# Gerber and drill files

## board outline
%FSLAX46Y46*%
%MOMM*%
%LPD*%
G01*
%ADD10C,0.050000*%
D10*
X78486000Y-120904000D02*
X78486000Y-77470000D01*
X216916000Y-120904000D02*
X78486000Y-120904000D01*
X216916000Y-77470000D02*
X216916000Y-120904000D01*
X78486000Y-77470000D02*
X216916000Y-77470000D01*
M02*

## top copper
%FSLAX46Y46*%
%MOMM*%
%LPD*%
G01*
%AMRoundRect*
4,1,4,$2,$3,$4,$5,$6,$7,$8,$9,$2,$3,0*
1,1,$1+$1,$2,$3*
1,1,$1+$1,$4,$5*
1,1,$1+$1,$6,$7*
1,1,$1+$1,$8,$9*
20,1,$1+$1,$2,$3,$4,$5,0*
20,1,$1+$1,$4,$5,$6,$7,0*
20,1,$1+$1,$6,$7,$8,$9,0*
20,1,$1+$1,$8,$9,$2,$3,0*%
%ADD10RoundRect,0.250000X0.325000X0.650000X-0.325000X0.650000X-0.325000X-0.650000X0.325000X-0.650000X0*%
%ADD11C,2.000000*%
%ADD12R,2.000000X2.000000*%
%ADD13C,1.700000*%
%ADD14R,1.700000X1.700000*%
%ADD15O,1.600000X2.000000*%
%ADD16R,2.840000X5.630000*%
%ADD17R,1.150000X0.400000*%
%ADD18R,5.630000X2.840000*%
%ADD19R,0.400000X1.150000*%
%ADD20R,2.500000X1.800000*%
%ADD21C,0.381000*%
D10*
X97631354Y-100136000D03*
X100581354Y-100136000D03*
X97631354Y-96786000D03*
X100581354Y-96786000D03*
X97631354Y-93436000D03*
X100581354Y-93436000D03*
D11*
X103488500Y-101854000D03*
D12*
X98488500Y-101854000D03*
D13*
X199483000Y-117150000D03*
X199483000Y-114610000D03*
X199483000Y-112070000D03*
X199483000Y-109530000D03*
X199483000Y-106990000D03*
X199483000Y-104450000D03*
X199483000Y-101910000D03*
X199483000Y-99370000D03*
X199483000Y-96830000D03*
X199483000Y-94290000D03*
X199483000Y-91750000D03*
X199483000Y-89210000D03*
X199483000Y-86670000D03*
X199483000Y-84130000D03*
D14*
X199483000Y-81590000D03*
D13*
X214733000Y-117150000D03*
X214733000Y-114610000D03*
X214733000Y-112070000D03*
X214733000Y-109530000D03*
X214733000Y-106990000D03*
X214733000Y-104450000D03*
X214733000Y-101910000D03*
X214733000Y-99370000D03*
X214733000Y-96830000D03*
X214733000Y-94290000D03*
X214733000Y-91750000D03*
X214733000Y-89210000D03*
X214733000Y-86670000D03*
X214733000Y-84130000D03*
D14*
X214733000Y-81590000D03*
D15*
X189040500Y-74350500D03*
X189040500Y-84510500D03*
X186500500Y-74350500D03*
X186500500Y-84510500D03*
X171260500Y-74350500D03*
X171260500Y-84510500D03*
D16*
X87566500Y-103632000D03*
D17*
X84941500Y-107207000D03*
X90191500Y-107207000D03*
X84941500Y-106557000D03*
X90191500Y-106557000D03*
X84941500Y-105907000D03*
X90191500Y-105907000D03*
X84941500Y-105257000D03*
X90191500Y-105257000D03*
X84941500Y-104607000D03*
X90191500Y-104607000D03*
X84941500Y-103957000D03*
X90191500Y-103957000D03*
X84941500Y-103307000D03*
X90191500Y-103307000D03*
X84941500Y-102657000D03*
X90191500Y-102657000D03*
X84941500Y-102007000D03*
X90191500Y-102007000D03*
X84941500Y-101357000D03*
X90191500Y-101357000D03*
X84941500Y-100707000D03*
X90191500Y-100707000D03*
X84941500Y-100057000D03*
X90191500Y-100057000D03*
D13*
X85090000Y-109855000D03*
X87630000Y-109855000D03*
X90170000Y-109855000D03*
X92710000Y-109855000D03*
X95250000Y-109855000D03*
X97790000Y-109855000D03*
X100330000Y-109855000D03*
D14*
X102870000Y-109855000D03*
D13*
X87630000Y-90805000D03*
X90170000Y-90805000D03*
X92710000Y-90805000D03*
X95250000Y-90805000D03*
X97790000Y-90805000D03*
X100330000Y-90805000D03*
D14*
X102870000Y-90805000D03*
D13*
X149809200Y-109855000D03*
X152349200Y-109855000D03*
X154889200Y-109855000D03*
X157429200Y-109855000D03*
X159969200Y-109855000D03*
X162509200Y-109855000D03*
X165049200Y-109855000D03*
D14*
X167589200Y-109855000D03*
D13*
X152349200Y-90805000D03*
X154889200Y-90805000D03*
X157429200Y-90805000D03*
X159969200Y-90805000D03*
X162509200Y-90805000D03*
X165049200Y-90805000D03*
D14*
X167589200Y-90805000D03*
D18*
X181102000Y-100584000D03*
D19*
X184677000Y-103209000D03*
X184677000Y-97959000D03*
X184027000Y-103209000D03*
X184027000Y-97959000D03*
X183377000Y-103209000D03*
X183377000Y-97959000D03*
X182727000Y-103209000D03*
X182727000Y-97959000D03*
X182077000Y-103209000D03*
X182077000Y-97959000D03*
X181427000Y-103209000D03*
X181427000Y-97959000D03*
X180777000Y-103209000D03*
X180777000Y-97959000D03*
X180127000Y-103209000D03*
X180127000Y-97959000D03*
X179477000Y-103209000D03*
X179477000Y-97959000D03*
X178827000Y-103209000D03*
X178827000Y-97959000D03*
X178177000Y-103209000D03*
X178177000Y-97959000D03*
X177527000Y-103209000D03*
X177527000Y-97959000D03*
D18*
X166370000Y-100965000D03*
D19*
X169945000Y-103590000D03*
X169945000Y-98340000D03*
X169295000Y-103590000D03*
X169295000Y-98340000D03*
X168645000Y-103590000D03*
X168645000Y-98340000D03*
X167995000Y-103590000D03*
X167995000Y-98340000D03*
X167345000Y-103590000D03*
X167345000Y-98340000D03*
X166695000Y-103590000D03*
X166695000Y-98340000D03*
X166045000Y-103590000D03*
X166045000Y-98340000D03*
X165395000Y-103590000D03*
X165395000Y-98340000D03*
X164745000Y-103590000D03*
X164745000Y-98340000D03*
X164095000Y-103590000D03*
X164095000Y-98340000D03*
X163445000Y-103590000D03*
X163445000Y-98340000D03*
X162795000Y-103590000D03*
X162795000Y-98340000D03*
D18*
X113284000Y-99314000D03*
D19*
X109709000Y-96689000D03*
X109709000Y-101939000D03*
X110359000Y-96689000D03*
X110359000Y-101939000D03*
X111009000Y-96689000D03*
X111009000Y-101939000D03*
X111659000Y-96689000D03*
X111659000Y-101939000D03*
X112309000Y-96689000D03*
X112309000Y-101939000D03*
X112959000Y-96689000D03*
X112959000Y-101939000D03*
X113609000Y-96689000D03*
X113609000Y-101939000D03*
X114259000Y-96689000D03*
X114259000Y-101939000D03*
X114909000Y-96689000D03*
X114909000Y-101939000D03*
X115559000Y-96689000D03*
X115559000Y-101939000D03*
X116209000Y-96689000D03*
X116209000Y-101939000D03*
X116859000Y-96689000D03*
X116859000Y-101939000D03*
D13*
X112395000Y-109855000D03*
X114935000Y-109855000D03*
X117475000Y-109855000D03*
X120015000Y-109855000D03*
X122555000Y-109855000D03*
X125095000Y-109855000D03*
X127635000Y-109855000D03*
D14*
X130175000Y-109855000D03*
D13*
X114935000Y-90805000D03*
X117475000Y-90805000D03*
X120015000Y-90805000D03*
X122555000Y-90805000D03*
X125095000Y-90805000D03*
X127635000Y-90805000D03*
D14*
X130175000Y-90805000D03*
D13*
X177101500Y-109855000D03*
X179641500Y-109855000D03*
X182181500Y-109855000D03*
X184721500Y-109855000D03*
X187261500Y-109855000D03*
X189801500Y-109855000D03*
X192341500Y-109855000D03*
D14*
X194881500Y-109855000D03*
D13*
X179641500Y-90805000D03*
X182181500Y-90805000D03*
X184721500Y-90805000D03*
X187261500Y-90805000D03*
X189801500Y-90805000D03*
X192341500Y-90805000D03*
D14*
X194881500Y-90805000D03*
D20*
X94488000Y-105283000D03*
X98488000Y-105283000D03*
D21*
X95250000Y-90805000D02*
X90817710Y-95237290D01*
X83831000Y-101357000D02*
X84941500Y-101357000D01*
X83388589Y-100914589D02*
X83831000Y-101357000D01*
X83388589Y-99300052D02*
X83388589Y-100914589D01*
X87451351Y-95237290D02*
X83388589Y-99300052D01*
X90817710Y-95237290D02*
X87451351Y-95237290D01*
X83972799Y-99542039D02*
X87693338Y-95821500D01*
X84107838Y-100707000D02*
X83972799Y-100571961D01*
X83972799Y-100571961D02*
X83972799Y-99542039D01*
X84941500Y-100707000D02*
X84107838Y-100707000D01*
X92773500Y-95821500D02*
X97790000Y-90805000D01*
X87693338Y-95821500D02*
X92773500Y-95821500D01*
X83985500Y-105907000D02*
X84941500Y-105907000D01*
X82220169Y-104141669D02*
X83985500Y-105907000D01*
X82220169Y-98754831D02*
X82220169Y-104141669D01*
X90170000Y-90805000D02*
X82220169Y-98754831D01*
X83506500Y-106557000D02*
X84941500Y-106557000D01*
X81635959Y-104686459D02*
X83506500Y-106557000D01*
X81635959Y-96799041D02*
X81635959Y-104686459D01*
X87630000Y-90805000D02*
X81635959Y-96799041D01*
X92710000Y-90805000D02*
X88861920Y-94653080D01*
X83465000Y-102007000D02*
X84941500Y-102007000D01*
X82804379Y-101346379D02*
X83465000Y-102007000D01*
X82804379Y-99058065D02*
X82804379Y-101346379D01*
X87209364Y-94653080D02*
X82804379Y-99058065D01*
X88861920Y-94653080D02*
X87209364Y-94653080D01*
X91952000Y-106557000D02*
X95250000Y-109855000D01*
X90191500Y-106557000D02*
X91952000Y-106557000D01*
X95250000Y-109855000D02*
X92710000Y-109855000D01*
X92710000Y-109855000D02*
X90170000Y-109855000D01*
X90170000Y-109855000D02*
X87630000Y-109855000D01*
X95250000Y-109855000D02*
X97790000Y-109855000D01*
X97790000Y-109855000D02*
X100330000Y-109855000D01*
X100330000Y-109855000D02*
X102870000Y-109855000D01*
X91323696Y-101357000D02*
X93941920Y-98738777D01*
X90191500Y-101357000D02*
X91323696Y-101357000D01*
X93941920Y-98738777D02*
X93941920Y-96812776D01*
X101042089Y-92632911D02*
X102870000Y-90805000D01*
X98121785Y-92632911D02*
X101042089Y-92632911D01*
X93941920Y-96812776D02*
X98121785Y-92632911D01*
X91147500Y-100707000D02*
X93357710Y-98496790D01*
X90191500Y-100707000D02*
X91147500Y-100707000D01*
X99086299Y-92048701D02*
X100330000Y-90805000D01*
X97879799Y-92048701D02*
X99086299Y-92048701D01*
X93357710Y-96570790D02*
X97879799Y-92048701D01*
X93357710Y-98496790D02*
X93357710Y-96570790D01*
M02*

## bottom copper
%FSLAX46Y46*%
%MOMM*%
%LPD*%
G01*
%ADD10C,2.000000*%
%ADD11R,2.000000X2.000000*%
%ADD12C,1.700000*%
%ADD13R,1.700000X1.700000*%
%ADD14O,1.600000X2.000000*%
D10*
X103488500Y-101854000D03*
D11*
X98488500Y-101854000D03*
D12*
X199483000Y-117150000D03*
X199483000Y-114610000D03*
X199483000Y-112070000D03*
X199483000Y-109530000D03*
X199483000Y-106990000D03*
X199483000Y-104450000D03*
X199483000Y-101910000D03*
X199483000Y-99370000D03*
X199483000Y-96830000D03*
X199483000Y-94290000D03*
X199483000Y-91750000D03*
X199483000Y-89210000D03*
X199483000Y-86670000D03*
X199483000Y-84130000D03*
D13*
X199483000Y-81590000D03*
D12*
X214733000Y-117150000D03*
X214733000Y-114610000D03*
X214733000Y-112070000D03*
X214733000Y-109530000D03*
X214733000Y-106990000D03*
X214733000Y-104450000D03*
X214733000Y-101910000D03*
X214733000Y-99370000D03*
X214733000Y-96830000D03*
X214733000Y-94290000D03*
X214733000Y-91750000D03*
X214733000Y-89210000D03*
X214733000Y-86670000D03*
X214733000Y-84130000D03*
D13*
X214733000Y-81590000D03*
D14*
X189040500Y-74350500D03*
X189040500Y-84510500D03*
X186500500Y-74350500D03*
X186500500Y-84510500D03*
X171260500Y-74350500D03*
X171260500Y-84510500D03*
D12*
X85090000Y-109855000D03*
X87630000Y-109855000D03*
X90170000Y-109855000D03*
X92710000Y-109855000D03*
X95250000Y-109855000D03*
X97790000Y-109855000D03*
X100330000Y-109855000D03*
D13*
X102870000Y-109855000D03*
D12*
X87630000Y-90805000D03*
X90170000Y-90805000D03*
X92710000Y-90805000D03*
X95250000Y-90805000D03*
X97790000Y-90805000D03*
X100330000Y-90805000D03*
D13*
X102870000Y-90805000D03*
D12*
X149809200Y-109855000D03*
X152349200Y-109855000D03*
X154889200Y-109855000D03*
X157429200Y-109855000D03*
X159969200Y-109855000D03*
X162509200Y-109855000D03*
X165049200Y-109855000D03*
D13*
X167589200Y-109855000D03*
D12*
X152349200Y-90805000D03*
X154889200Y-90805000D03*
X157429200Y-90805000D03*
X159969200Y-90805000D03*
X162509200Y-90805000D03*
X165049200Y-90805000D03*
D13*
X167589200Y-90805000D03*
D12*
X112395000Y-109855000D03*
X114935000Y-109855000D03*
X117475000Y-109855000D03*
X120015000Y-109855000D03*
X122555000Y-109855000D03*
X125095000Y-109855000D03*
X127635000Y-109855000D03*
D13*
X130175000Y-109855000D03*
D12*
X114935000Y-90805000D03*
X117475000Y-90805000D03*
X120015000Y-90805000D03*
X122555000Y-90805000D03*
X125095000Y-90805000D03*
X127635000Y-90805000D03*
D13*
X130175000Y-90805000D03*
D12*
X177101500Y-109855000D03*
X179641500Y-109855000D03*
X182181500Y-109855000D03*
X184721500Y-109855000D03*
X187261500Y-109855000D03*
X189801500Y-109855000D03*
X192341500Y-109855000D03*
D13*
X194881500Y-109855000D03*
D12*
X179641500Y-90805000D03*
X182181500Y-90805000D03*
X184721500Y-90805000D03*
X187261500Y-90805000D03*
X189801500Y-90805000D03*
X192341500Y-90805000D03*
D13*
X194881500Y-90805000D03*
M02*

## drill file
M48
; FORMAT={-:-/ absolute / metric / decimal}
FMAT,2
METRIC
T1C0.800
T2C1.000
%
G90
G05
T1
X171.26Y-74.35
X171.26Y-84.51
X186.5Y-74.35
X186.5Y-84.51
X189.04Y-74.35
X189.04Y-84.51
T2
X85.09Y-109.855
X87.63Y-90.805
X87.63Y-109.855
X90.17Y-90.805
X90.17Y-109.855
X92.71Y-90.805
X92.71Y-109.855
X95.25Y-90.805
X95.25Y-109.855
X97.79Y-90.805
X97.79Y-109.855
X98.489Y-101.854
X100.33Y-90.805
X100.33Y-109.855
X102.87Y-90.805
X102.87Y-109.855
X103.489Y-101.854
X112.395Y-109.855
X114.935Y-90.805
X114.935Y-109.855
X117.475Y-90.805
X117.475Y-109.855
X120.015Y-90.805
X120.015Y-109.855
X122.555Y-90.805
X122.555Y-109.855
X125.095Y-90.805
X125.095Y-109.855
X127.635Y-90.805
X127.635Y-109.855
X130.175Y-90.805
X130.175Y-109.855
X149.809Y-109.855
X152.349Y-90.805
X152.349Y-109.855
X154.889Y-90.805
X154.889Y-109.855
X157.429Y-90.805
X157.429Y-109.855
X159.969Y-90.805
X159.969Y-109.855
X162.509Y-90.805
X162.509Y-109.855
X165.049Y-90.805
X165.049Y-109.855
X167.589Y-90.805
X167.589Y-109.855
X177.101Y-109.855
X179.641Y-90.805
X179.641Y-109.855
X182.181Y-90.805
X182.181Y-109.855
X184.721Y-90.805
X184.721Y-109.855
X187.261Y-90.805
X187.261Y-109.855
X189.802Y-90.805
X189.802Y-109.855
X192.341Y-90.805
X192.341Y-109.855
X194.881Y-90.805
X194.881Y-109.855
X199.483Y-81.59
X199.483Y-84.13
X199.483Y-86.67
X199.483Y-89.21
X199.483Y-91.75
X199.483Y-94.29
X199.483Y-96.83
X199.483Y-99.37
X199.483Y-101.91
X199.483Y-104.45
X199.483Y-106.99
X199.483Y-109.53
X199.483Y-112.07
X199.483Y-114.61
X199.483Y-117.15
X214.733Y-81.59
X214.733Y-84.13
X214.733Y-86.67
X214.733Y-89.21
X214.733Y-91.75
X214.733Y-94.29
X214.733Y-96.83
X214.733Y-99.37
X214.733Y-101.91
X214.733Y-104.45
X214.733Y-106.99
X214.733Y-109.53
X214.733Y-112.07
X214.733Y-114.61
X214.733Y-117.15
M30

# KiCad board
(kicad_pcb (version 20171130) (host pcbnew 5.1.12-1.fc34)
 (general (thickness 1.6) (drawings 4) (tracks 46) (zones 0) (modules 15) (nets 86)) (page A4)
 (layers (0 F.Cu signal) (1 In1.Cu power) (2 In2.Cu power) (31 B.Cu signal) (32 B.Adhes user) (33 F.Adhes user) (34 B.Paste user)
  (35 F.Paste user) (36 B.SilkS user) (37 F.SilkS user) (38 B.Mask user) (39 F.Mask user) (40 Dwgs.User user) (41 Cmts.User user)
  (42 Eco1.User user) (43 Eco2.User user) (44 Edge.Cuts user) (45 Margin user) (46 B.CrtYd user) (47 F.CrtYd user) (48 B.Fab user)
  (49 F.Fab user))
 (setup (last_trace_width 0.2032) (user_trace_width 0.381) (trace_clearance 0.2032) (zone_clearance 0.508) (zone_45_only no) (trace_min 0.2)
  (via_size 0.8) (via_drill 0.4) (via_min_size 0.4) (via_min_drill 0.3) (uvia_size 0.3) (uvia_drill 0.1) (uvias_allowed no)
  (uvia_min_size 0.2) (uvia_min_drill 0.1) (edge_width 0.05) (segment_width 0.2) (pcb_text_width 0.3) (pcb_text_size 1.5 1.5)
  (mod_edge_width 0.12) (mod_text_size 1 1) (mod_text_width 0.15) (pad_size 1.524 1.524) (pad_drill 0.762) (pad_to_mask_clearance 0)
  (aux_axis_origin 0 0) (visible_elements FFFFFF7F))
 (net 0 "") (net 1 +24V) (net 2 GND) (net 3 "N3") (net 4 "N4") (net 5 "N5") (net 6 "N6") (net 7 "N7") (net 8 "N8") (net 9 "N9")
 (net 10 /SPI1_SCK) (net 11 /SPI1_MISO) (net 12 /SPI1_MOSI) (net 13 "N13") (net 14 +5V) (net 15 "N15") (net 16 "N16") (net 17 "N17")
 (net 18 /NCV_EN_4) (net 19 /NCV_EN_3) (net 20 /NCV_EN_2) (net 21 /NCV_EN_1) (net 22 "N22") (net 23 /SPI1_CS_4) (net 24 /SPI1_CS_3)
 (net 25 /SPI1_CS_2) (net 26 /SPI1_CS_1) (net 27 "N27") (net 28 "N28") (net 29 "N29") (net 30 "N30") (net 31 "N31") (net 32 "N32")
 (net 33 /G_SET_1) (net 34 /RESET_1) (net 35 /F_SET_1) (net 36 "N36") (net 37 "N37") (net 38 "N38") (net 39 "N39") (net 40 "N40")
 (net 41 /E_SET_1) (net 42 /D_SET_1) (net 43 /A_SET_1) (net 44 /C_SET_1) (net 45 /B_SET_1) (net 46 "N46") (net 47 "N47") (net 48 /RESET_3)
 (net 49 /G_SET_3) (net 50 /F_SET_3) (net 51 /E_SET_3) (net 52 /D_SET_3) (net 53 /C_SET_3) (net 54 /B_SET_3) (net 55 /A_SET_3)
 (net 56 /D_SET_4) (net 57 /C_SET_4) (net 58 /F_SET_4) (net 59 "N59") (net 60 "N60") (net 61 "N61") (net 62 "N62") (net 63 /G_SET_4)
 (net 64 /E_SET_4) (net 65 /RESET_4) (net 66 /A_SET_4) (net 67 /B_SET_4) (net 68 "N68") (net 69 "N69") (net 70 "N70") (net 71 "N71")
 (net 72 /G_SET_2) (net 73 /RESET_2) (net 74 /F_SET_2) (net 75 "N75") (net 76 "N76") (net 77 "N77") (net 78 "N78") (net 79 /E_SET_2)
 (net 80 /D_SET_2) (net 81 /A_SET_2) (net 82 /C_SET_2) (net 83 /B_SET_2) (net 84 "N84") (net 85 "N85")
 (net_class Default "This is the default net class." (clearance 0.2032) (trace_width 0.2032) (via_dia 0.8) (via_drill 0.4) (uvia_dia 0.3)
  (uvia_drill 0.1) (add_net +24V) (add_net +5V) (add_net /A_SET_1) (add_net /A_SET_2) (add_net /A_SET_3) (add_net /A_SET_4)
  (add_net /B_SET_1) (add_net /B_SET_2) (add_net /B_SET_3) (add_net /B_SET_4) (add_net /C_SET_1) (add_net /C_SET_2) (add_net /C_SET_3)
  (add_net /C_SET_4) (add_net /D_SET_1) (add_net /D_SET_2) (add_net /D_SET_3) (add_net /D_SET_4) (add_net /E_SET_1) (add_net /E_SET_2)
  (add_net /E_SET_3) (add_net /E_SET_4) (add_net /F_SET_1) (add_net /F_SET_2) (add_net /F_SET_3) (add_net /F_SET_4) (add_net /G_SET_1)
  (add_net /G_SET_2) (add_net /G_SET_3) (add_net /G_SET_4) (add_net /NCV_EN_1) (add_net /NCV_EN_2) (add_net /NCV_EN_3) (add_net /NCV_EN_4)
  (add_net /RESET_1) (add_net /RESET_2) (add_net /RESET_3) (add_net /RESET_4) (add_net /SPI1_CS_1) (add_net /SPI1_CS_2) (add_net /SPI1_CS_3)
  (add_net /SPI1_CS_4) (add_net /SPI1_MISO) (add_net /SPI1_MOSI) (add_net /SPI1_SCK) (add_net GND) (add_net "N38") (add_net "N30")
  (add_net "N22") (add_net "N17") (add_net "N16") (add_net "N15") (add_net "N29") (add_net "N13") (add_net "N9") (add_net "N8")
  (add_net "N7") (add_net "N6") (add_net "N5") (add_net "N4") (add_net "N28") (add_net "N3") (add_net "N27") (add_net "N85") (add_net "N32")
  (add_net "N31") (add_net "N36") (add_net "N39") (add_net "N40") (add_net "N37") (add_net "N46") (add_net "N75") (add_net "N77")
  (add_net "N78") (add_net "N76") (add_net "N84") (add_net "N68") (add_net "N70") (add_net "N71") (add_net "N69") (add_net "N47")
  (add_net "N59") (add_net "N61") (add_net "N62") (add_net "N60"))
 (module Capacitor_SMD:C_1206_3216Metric (layer F.Cu) (at 99.106354 100.136 180)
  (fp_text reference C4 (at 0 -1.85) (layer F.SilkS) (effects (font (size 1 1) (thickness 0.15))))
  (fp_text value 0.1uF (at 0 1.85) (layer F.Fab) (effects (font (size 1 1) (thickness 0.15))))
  (pad 2 smd roundrect (at 1.475 0 180) (size 1.15 1.8) (layers F.Cu F.Paste F.Mask) (roundrect_rratio 0.217391) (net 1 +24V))
  (pad 1 smd roundrect (at -1.475 0 180) (size 1.15 1.8) (layers F.Cu F.Paste F.Mask) (roundrect_rratio 0.217391) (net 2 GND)))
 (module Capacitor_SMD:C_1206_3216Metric (layer F.Cu) (at 99.106354 96.786 180)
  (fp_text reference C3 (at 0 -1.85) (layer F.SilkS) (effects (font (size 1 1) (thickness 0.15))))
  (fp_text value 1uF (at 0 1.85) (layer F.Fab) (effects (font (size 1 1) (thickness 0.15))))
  (pad 2 smd roundrect (at 1.475 0 180) (size 1.15 1.8) (layers F.Cu F.Paste F.Mask) (roundrect_rratio 0.217391) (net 1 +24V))
  (pad 1 smd roundrect (at -1.475 0 180) (size 1.15 1.8) (layers F.Cu F.Paste F.Mask) (roundrect_rratio 0.217391) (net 2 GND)))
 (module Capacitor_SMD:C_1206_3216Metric (layer F.Cu) (at 99.106354 93.436 180)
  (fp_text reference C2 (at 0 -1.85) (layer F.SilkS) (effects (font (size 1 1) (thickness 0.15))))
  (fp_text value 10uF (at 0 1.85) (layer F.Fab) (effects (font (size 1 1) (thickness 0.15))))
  (pad 2 smd roundrect (at 1.475 0 180) (size 1.15 1.8) (layers F.Cu F.Paste F.Mask) (roundrect_rratio 0.217391) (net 1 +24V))
  (pad 1 smd roundrect (at -1.475 0 180) (size 1.15 1.8) (layers F.Cu F.Paste F.Mask) (roundrect_rratio 0.217391) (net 2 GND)))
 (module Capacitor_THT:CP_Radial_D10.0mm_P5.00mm (layer B.Cu) (at 98.4885 101.854)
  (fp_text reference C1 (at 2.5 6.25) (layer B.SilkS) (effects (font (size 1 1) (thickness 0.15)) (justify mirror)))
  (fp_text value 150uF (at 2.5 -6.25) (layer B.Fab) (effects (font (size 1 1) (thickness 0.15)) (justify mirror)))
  (pad 2 thru_hole circle (at 5 0) (size 2 2) (drill 1) (layers *.Cu *.Mask) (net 2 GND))
  (pad 1 thru_hole rect (at 0 0) (size 2 2) (drill 1) (layers *.Cu *.Mask) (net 1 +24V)))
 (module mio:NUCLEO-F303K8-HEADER (layer B.Cu) (at 216.408 123.19 180)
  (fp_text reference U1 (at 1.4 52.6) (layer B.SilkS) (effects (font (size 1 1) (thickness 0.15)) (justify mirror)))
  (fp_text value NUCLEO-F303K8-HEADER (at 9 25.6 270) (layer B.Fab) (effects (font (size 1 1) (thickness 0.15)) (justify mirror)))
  (pad 30 thru_hole circle (at 16.925 6.04 180) (size 1.7 1.7) (drill 1) (layers *.Cu *.Mask) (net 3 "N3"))
  (pad 29 thru_hole circle (at 16.925 8.58 180) (size 1.7 1.7) (drill 1) (layers *.Cu *.Mask) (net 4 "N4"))
  (pad 28 thru_hole circle (at 16.925 11.12 180) (size 1.7 1.7) (drill 1) (layers *.Cu *.Mask) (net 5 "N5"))
  (pad 27 thru_hole circle (at 16.925 13.66 180) (size 1.7 1.7) (drill 1) (layers *.Cu *.Mask) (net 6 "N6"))
  (pad 26 thru_hole circle (at 16.925 16.2 180) (size 1.7 1.7) (drill 1) (layers *.Cu *.Mask) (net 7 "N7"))
  (pad 25 thru_hole circle (at 16.925 18.74 180) (size 1.7 1.7) (drill 1) (layers *.Cu *.Mask) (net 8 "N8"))
  (pad 24 thru_hole circle (at 16.925 21.28 180) (size 1.7 1.7) (drill 1) (layers *.Cu *.Mask) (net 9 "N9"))
  (pad 23 thru_hole circle (at 16.925 23.82 180) (size 1.7 1.7) (drill 1) (layers *.Cu *.Mask) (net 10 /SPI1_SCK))
  (pad 22 thru_hole circle (at 16.925 26.36 180) (size 1.7 1.7) (drill 1) (layers *.Cu *.Mask) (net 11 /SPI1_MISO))
  (pad 21 thru_hole circle (at 16.925 28.9 180) (size 1.7 1.7) (drill 1) (layers *.Cu *.Mask) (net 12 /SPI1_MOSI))
  (pad 20 thru_hole circle (at 16.925 31.44 180) (size 1.7 1.7) (drill 1) (layers *.Cu *.Mask) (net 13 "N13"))
  (pad 19 thru_hole circle (at 16.925 33.98 180) (size 1.7 1.7) (drill 1) (layers *.Cu *.Mask) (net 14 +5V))
  (pad 18 thru_hole circle (at 16.925 36.52 180) (size 1.7 1.7) (drill 1) (layers *.Cu *.Mask) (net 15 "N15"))
  (pad 17 thru_hole circle (at 16.925 39.06 180) (size 1.7 1.7) (drill 1) (layers *.Cu *.Mask) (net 2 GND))
  (pad 16 thru_hole rect (at 16.925 41.6 180) (size 1.7 1.7) (drill 1) (layers *.Cu *.Mask) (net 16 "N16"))
  (pad 15 thru_hole circle (at 1.675 6.04 180) (size 1.7 1.7) (drill 1) (layers *.Cu *.Mask) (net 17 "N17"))
  (pad 14 thru_hole circle (at 1.675 8.58 180) (size 1.7 1.7) (drill 1) (layers *.Cu *.Mask) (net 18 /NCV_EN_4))
  (pad 13 thru_hole circle (at 1.675 11.12 180) (size 1.7 1.7) (drill 1) (layers *.Cu *.Mask) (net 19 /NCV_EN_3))
  (pad 12 thru_hole circle (at 1.675 13.66 180) (size 1.7 1.7) (drill 1) (layers *.Cu *.Mask) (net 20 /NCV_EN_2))
  (pad 11 thru_hole circle (at 1.675 16.2 180) (size 1.7 1.7) (drill 1) (layers *.Cu *.Mask) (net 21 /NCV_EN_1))
  (pad 10 thru_hole circle (at 1.675 18.74 180) (size 1.7 1.7) (drill 1) (layers *.Cu *.Mask) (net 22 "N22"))
  (pad 9 thru_hole circle (at 1.675 21.28 180) (size 1.7 1.7) (drill 1) (layers *.Cu *.Mask) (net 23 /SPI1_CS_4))
  (pad 8 thru_hole circle (at 1.675 23.82 180) (size 1.7 1.7) (drill 1) (layers *.Cu *.Mask) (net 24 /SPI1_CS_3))
  (pad 7 thru_hole circle (at 1.675 26.36 180) (size 1.7 1.7) (drill 1) (layers *.Cu *.Mask) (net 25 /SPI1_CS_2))
  (pad 6 thru_hole circle (at 1.675 28.9 180) (size 1.7 1.7) (drill 1) (layers *.Cu *.Mask) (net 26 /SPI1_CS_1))
  (pad 5 thru_hole circle (at 1.675 31.44 180) (size 1.7 1.7) (drill 1) (layers *.Cu *.Mask) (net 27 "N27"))
  (pad 4 thru_hole circle (at 1.675 33.98 180) (size 1.7 1.7) (drill 1) (layers *.Cu *.Mask) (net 2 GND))
  (pad 3 thru_hole circle (at 1.675 36.52 180) (size 1.7 1.7) (drill 1) (layers *.Cu *.Mask) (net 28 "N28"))
  (pad 2 thru_hole circle (at 1.675 39.06 180) (size 1.7 1.7) (drill 1) (layers *.Cu *.Mask) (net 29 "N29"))
  (pad 1 thru_hole rect (at 1.675 41.6 180) (size 1.7 1.7) (drill 1) (layers *.Cu *.Mask) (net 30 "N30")))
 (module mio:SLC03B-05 (layer B.Cu) (at 169.1005 72.5805)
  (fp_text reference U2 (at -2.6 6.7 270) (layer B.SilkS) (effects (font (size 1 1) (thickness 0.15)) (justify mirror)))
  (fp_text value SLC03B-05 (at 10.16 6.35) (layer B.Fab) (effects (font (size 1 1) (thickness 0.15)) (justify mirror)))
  (pad 8 thru_hole oval (at 19.94 1.77) (size 1.6 2) (drill 0.8) (layers *.Cu *.Mask) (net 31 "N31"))
  (pad 9 thru_hole oval (at 19.94 11.93) (size 1.6 2) (drill 0.8) (layers *.Cu *.Mask) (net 14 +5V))
  (pad 7 thru_hole oval (at 17.4 1.77) (size 1.6 2) (drill 0.8) (layers *.Cu *.Mask) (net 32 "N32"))
  (pad 10 thru_hole oval (at 17.4 11.93) (size 1.6 2) (drill 0.8) (layers *.Cu *.Mask) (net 2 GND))
  (pad 1 thru_hole oval (at 2.16 1.77) (size 1.6 2) (drill 0.8) (layers *.Cu *.Mask) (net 2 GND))
  (pad 16 thru_hole oval (at 2.16 11.93) (size 1.6 2) (drill 0.8) (layers *.Cu *.Mask) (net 1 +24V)))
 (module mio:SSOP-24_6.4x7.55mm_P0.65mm (layer F.Cu) (at 87.5665 103.632 270)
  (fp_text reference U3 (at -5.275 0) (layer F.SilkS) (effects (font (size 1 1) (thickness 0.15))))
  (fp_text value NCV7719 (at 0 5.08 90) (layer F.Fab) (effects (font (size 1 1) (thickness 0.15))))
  (pad 25 smd rect (at 0 0 270) (size 5.63 2.84) (layers F.Cu F.Paste F.Mask) (zone_connect 1) (thermal_width 0.5) (thermal_gap 0.5))
  (pad 12 smd rect (at 3.575 2.625 270) (size 0.4 1.15) (layers F.Cu F.Paste F.Mask) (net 2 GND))
  (pad 13 smd rect (at 3.575 -2.625 270) (size 0.4 1.15) (layers F.Cu F.Paste F.Mask) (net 2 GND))
  (pad 11 smd rect (at 2.925 2.625 270) (size 0.4 1.15) (layers F.Cu F.Paste F.Mask) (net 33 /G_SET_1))
  (pad 14 smd rect (at 2.925 -2.625 270) (size 0.4 1.15) (layers F.Cu F.Paste F.Mask) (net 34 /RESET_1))
  (pad 10 smd rect (at 2.275 2.625 270) (size 0.4 1.15) (layers F.Cu F.Paste F.Mask) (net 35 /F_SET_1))
  (pad 15 smd rect (at 2.275 -2.625 270) (size 0.4 1.15) (layers F.Cu F.Paste F.Mask) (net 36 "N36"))
  (pad 9 smd rect (at 1.625 2.625 270) (size 0.4 1.15) (layers F.Cu F.Paste F.Mask) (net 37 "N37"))
  (pad 16 smd rect (at 1.625 -2.625 270) (size 0.4 1.15) (layers F.Cu F.Paste F.Mask) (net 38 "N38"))
  (pad 8 smd rect (at 0.975 2.625 270) (size 0.4 1.15) (layers F.Cu F.Paste F.Mask) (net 21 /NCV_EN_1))
  (pad 17 smd rect (at 0.975 -2.625 270) (size 0.4 1.15) (layers F.Cu F.Paste F.Mask) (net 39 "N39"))
  (pad 7 smd rect (at 0.325 2.625 270) (size 0.4 1.15) (layers F.Cu F.Paste F.Mask) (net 11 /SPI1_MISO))
  (pad 18 smd rect (at 0.325 -2.625 270) (size 0.4 1.15) (layers F.Cu F.Paste F.Mask) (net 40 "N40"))
  (pad 6 smd rect (at -0.325 2.625 270) (size 0.4 1.15) (layers F.Cu F.Paste F.Mask) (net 14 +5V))
  (pad 19 smd rect (at -0.325 -2.625 270) (size 0.4 1.15) (layers F.Cu F.Paste F.Mask) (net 26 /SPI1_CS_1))
  (pad 5 smd rect (at -0.975 2.625 270) (size 0.4 1.15) (layers F.Cu F.Paste F.Mask) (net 12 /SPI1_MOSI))
  (pad 20 smd rect (at -0.975 -2.625 270) (size 0.4 1.15) (layers F.Cu F.Paste F.Mask) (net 10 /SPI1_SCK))
  (pad 4 smd rect (at -1.625 2.625 270) (size 0.4 1.15) (layers F.Cu F.Paste F.Mask) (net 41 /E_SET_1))
  (pad 21 smd rect (at -1.625 -2.625 270) (size 0.4 1.15) (layers F.Cu F.Paste F.Mask) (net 38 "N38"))
  (pad 3 smd rect (at -2.275 2.625 270) (size 0.4 1.15) (layers F.Cu F.Paste F.Mask) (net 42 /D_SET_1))
  (pad 22 smd rect (at -2.275 -2.625 270) (size 0.4 1.15) (layers F.Cu F.Paste F.Mask) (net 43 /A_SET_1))
  (pad 2 smd rect (at -2.925 2.625 270) (size 0.4 1.15) (layers F.Cu F.Paste F.Mask) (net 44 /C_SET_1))
  (pad 23 smd rect (at -2.925 -2.625 270) (size 0.4 1.15) (layers F.Cu F.Paste F.Mask) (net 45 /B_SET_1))
  (pad 1 smd rect (at -3.575 2.625 270) (size 0.4 1.15) (layers F.Cu F.Paste F.Mask) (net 2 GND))
  (pad 24 smd rect (at -3.575 -2.625 270) (size 0.4 1.15) (layers F.Cu F.Paste F.Mask) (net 2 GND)))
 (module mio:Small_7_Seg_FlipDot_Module (layer F.Cu) (at 81.28 116.205)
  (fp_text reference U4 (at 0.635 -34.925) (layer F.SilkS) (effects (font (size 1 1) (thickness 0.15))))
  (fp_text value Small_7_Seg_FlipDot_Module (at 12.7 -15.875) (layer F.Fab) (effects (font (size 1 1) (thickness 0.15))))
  (pad 15 thru_hole circle (at 3.81 -6.35) (size 1.7 1.7) (drill 1) (layers *.Cu *.Mask) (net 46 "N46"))
  (pad 14 thru_hole circle (at 6.35 -6.35) (size 1.7 1.7) (drill 1) (layers *.Cu *.Mask) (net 34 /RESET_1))
  (pad 13 thru_hole circle (at 8.89 -6.35) (size 1.7 1.7) (drill 1) (layers *.Cu *.Mask) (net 34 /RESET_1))
  (pad 12 thru_hole circle (at 11.43 -6.35) (size 1.7 1.7) (drill 1) (layers *.Cu *.Mask) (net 34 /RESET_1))
  (pad 11 thru_hole circle (at 13.97 -6.35) (size 1.7 1.7) (drill 1) (layers *.Cu *.Mask) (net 34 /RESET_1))
  (pad 10 thru_hole circle (at 16.51 -6.35) (size 1.7 1.7) (drill 1) (layers *.Cu *.Mask) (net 34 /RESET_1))
  (pad 9 thru_hole circle (at 19.05 -6.35) (size 1.7 1.7) (drill 1) (layers *.Cu *.Mask) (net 34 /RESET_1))
  (pad 8 thru_hole rect (at 21.59 -6.35) (size 1.7 1.7) (drill 1) (layers *.Cu *.Mask) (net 34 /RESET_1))
  (pad 7 thru_hole circle (at 6.35 -25.4) (size 1.7 1.7) (drill 1) (layers *.Cu *.Mask) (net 33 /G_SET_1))
  (pad 6 thru_hole circle (at 8.89 -25.4) (size 1.7 1.7) (drill 1) (layers *.Cu *.Mask) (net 35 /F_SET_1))
  (pad 5 thru_hole circle (at 11.43 -25.4) (size 1.7 1.7) (drill 1) (layers *.Cu *.Mask) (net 41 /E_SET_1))
  (pad 4 thru_hole circle (at 13.97 -25.4) (size 1.7 1.7) (drill 1) (layers *.Cu *.Mask) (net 42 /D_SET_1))
  (pad 3 thru_hole circle (at 16.51 -25.4) (size 1.7 1.7) (drill 1) (layers *.Cu *.Mask) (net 44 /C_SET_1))
  (pad 2 thru_hole circle (at 19.05 -25.4) (size 1.7 1.7) (drill 1) (layers *.Cu *.Mask) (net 45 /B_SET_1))
  (pad 1 thru_hole rect (at 21.59 -25.4) (size 1.7 1.7) (drill 1) (layers *.Cu *.Mask) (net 43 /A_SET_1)))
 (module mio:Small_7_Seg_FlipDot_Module (layer F.Cu) (at 145.9992 116.205)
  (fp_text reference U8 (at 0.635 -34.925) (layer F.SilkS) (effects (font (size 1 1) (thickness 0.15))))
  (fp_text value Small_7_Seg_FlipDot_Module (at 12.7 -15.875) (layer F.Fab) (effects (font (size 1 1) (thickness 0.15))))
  (pad 15 thru_hole circle (at 3.81 -6.35) (size 1.7 1.7) (drill 1) (layers *.Cu *.Mask) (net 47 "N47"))
  (pad 14 thru_hole circle (at 6.35 -6.35) (size 1.7 1.7) (drill 1) (layers *.Cu *.Mask) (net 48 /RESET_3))
  (pad 13 thru_hole circle (at 8.89 -6.35) (size 1.7 1.7) (drill 1) (layers *.Cu *.Mask) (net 48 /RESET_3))
  (pad 12 thru_hole circle (at 11.43 -6.35) (size 1.7 1.7) (drill 1) (layers *.Cu *.Mask) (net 48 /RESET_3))
  (pad 11 thru_hole circle (at 13.97 -6.35) (size 1.7 1.7) (drill 1) (layers *.Cu *.Mask) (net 48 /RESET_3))
  (pad 10 thru_hole circle (at 16.51 -6.35) (size 1.7 1.7) (drill 1) (layers *.Cu *.Mask) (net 48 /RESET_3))
  (pad 9 thru_hole circle (at 19.05 -6.35) (size 1.7 1.7) (drill 1) (layers *.Cu *.Mask) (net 48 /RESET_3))
  (pad 8 thru_hole rect (at 21.59 -6.35) (size 1.7 1.7) (drill 1) (layers *.Cu *.Mask) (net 48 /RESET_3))
  (pad 7 thru_hole circle (at 6.35 -25.4) (size 1.7 1.7) (drill 1) (layers *.Cu *.Mask) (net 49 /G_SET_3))
  (pad 6 thru_hole circle (at 8.89 -25.4) (size 1.7 1.7) (drill 1) (layers *.Cu *.Mask) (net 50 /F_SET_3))
  (pad 5 thru_hole circle (at 11.43 -25.4) (size 1.7 1.7) (drill 1) (layers *.Cu *.Mask) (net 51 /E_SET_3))
  (pad 4 thru_hole circle (at 13.97 -25.4) (size 1.7 1.7) (drill 1) (layers *.Cu *.Mask) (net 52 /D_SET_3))
  (pad 3 thru_hole circle (at 16.51 -25.4) (size 1.7 1.7) (drill 1) (layers *.Cu *.Mask) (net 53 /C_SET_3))
  (pad 2 thru_hole circle (at 19.05 -25.4) (size 1.7 1.7) (drill 1) (layers *.Cu *.Mask) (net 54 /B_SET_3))
  (pad 1 thru_hole rect (at 21.59 -25.4) (size 1.7 1.7) (drill 1) (layers *.Cu *.Mask) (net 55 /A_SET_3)))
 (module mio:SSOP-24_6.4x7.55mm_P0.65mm (layer F.Cu) (at 181.102 100.584)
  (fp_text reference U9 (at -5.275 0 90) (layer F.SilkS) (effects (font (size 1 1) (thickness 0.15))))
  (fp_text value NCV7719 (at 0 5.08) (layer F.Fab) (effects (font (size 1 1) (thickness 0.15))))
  (pad 25 smd rect (at 0 0) (size 5.63 2.84) (layers F.Cu F.Paste F.Mask) (zone_connect 1) (thermal_width 0.5) (thermal_gap 0.5))
  (pad 12 smd rect (at 3.575 2.625) (size 0.4 1.15) (layers F.Cu F.Paste F.Mask) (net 2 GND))
  (pad 13 smd rect (at 3.575 -2.625) (size 0.4 1.15) (layers F.Cu F.Paste F.Mask) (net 2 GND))
  (pad 11 smd rect (at 2.925 2.625) (size 0.4 1.15) (layers F.Cu F.Paste F.Mask) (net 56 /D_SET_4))
  (pad 14 smd rect (at 2.925 -2.625) (size 0.4 1.15) (layers F.Cu F.Paste F.Mask) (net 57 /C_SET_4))
  (pad 10 smd rect (at 2.275 2.625) (size 0.4 1.15) (layers F.Cu F.Paste F.Mask) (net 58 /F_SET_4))
  (pad 15 smd rect (at 2.275 -2.625) (size 0.4 1.15) (layers F.Cu F.Paste F.Mask) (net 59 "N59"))
  (pad 9 smd rect (at 1.625 2.625) (size 0.4 1.15) (layers F.Cu F.Paste F.Mask) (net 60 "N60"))
  (pad 16 smd rect (at 1.625 -2.625) (size 0.4 1.15) (layers F.Cu F.Paste F.Mask) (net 1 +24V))
  (pad 8 smd rect (at 0.975 2.625) (size 0.4 1.15) (layers F.Cu F.Paste F.Mask) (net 18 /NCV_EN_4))
  (pad 17 smd rect (at 0.975 -2.625) (size 0.4 1.15) (layers F.Cu F.Paste F.Mask) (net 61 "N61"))
  (pad 7 smd rect (at 0.325 2.625) (size 0.4 1.15) (layers F.Cu F.Paste F.Mask) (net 11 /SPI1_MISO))
  (pad 18 smd rect (at 0.325 -2.625) (size 0.4 1.15) (layers F.Cu F.Paste F.Mask) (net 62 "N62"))
  (pad 6 smd rect (at -0.325 2.625) (size 0.4 1.15) (layers F.Cu F.Paste F.Mask) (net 14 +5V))
  (pad 19 smd rect (at -0.325 -2.625) (size 0.4 1.15) (layers F.Cu F.Paste F.Mask) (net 23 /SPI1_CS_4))
  (pad 5 smd rect (at -0.975 2.625) (size 0.4 1.15) (layers F.Cu F.Paste F.Mask) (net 12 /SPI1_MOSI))
  (pad 20 smd rect (at -0.975 -2.625) (size 0.4 1.15) (layers F.Cu F.Paste F.Mask) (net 10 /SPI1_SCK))
  (pad 4 smd rect (at -1.625 2.625) (size 0.4 1.15) (layers F.Cu F.Paste F.Mask) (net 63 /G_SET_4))
  (pad 21 smd rect (at -1.625 -2.625) (size 0.4 1.15) (layers F.Cu F.Paste F.Mask) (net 1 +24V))
  (pad 3 smd rect (at -2.275 2.625) (size 0.4 1.15) (layers F.Cu F.Paste F.Mask) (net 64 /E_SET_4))
  (pad 22 smd rect (at -2.275 -2.625) (size 0.4 1.15) (layers F.Cu F.Paste F.Mask) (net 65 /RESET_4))
  (pad 2 smd rect (at -2.925 2.625) (size 0.4 1.15) (layers F.Cu F.Paste F.Mask) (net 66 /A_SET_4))
  (pad 23 smd rect (at -2.925 -2.625) (size 0.4 1.15) (layers F.Cu F.Paste F.Mask) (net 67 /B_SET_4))
  (pad 1 smd rect (at -3.575 2.625) (size 0.4 1.15) (layers F.Cu F.Paste F.Mask) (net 2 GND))
  (pad 24 smd rect (at -3.575 -2.625) (size 0.4 1.15) (layers F.Cu F.Paste F.Mask) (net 2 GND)))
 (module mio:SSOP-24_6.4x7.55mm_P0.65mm (layer F.Cu) (at 166.37 100.965)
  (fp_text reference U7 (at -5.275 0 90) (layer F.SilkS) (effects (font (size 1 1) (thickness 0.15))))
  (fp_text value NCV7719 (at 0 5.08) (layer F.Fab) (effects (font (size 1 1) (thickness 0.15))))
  (pad 25 smd rect (at 0 0) (size 5.63 2.84) (layers F.Cu F.Paste F.Mask) (zone_connect 1) (thermal_width 0.5) (thermal_gap 0.5))
  (pad 12 smd rect (at 3.575 2.625) (size 0.4 1.15) (layers F.Cu F.Paste F.Mask) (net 2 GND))
  (pad 13 smd rect (at 3.575 -2.625) (size 0.4 1.15) (layers F.Cu F.Paste F.Mask) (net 2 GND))
  (pad 11 smd rect (at 2.925 2.625) (size 0.4 1.15) (layers F.Cu F.Paste F.Mask) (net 52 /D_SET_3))
  (pad 14 smd rect (at 2.925 -2.625) (size 0.4 1.15) (layers F.Cu F.Paste F.Mask) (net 53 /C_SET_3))
  (pad 10 smd rect (at 2.275 2.625) (size 0.4 1.15) (layers F.Cu F.Paste F.Mask) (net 50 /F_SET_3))
  (pad 15 smd rect (at 2.275 -2.625) (size 0.4 1.15) (layers F.Cu F.Paste F.Mask) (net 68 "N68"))
  (pad 9 smd rect (at 1.625 2.625) (size 0.4 1.15) (layers F.Cu F.Paste F.Mask) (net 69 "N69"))
  (pad 16 smd rect (at 1.625 -2.625) (size 0.4 1.15) (layers F.Cu F.Paste F.Mask) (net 1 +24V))
  (pad 8 smd rect (at 0.975 2.625) (size 0.4 1.15) (layers F.Cu F.Paste F.Mask) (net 19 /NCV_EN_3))
  (pad 17 smd rect (at 0.975 -2.625) (size 0.4 1.15) (layers F.Cu F.Paste F.Mask) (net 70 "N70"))
  (pad 7 smd rect (at 0.325 2.625) (size 0.4 1.15) (layers F.Cu F.Paste F.Mask) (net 11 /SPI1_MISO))
  (pad 18 smd rect (at 0.325 -2.625) (size 0.4 1.15) (layers F.Cu F.Paste F.Mask) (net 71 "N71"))
  (pad 6 smd rect (at -0.325 2.625) (size 0.4 1.15) (layers F.Cu F.Paste F.Mask) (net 14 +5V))
  (pad 19 smd rect (at -0.325 -2.625) (size 0.4 1.15) (layers F.Cu F.Paste F.Mask) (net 24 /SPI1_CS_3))
  (pad 5 smd rect (at -0.975 2.625) (size 0.4 1.15) (layers F.Cu F.Paste F.Mask) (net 12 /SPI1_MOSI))
  (pad 20 smd rect (at -0.975 -2.625) (size 0.4 1.15) (layers F.Cu F.Paste F.Mask) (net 10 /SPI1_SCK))
  (pad 4 smd rect (at -1.625 2.625) (size 0.4 1.15) (layers F.Cu F.Paste F.Mask) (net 49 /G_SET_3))
  (pad 21 smd rect (at -1.625 -2.625) (size 0.4 1.15) (layers F.Cu F.Paste F.Mask) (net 1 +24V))
  (pad 3 smd rect (at -2.275 2.625) (size 0.4 1.15) (layers F.Cu F.Paste F.Mask) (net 51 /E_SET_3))
  (pad 22 smd rect (at -2.275 -2.625) (size 0.4 1.15) (layers F.Cu F.Paste F.Mask) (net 48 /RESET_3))
  (pad 2 smd rect (at -2.925 2.625) (size 0.4 1.15) (layers F.Cu F.Paste F.Mask) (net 55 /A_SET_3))
  (pad 23 smd rect (at -2.925 -2.625) (size 0.4 1.15) (layers F.Cu F.Paste F.Mask) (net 54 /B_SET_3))
  (pad 1 smd rect (at -3.575 2.625) (size 0.4 1.15) (layers F.Cu F.Paste F.Mask) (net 2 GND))
  (pad 24 smd rect (at -3.575 -2.625) (size 0.4 1.15) (layers F.Cu F.Paste F.Mask) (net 2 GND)))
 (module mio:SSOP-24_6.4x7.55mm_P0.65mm (layer F.Cu) (at 113.284 99.314 180)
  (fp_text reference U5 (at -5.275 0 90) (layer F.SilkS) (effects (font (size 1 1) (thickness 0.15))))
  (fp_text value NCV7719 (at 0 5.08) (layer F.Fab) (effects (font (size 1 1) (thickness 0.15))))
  (pad 25 smd rect (at 0 0 180) (size 5.63 2.84) (layers F.Cu F.Paste F.Mask) (zone_connect 1) (thermal_width 0.5) (thermal_gap 0.5))
  (pad 12 smd rect (at 3.575 2.625 180) (size 0.4 1.15) (layers F.Cu F.Paste F.Mask) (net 2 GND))
  (pad 13 smd rect (at 3.575 -2.625 180) (size 0.4 1.15) (layers F.Cu F.Paste F.Mask) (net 2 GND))
  (pad 11 smd rect (at 2.925 2.625 180) (size 0.4 1.15) (layers F.Cu F.Paste F.Mask) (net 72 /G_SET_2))
  (pad 14 smd rect (at 2.925 -2.625 180) (size 0.4 1.15) (layers F.Cu F.Paste F.Mask) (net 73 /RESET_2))
  (pad 10 smd rect (at 2.275 2.625 180) (size 0.4 1.15) (layers F.Cu F.Paste F.Mask) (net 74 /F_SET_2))
  (pad 15 smd rect (at 2.275 -2.625 180) (size 0.4 1.15) (layers F.Cu F.Paste F.Mask) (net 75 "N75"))
  (pad 9 smd rect (at 1.625 2.625 180) (size 0.4 1.15) (layers F.Cu F.Paste F.Mask) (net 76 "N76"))
  (pad 16 smd rect (at 1.625 -2.625 180) (size 0.4 1.15) (layers F.Cu F.Paste F.Mask) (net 1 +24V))
  (pad 8 smd rect (at 0.975 2.625 180) (size 0.4 1.15) (layers F.Cu F.Paste F.Mask) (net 20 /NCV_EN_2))
  (pad 17 smd rect (at 0.975 -2.625 180) (size 0.4 1.15) (layers F.Cu F.Paste F.Mask) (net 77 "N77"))
  (pad 7 smd rect (at 0.325 2.625 180) (size 0.4 1.15) (layers F.Cu F.Paste F.Mask) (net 11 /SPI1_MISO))
  (pad 18 smd rect (at 0.325 -2.625 180) (size 0.4 1.15) (layers F.Cu F.Paste F.Mask) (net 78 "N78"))
  (pad 6 smd rect (at -0.325 2.625 180) (size 0.4 1.15) (layers F.Cu F.Paste F.Mask) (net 14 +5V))
  (pad 19 smd rect (at -0.325 -2.625 180) (size 0.4 1.15) (layers F.Cu F.Paste F.Mask) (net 25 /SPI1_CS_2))
  (pad 5 smd rect (at -0.975 2.625 180) (size 0.4 1.15) (layers F.Cu F.Paste F.Mask) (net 12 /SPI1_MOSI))
  (pad 20 smd rect (at -0.975 -2.625 180) (size 0.4 1.15) (layers F.Cu F.Paste F.Mask) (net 10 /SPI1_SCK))
  (pad 4 smd rect (at -1.625 2.625 180) (size 0.4 1.15) (layers F.Cu F.Paste F.Mask) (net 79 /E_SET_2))
  (pad 21 smd rect (at -1.625 -2.625 180) (size 0.4 1.15) (layers F.Cu F.Paste F.Mask) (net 1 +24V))
  (pad 3 smd rect (at -2.275 2.625 180) (size 0.4 1.15) (layers F.Cu F.Paste F.Mask) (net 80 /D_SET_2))
  (pad 22 smd rect (at -2.275 -2.625 180) (size 0.4 1.15) (layers F.Cu F.Paste F.Mask) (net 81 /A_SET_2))
  (pad 2 smd rect (at -2.925 2.625 180) (size 0.4 1.15) (layers F.Cu F.Paste F.Mask) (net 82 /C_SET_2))
  (pad 23 smd rect (at -2.925 -2.625 180) (size 0.4 1.15) (layers F.Cu F.Paste F.Mask) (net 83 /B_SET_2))
  (pad 1 smd rect (at -3.575 2.625 180) (size 0.4 1.15) (layers F.Cu F.Paste F.Mask) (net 2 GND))
  (pad 24 smd rect (at -3.575 -2.625 180) (size 0.4 1.15) (layers F.Cu F.Paste F.Mask) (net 2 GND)))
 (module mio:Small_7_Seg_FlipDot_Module (layer F.Cu) (at 108.585 116.205)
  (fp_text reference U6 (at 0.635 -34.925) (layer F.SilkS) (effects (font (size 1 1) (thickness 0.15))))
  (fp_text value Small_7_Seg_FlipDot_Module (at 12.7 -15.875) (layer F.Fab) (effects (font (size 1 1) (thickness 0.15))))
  (pad 15 thru_hole circle (at 3.81 -6.35) (size 1.7 1.7) (drill 1) (layers *.Cu *.Mask) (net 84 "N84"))
  (pad 14 thru_hole circle (at 6.35 -6.35) (size 1.7 1.7) (drill 1) (layers *.Cu *.Mask) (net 73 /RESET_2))
  (pad 13 thru_hole circle (at 8.89 -6.35) (size 1.7 1.7) (drill 1) (layers *.Cu *.Mask) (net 73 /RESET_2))
  (pad 12 thru_hole circle (at 11.43 -6.35) (size 1.7 1.7) (drill 1) (layers *.Cu *.Mask) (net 73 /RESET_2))
  (pad 11 thru_hole circle (at 13.97 -6.35) (size 1.7 1.7) (drill 1) (layers *.Cu *.Mask) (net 73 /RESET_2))
  (pad 10 thru_hole circle (at 16.51 -6.35) (size 1.7 1.7) (drill 1) (layers *.Cu *.Mask) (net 73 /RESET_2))
  (pad 9 thru_hole circle (at 19.05 -6.35) (size 1.7 1.7) (drill 1) (layers *.Cu *.Mask) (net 73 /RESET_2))
  (pad 8 thru_hole rect (at 21.59 -6.35) (size 1.7 1.7) (drill 1) (layers *.Cu *.Mask) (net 73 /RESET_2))
  (pad 7 thru_hole circle (at 6.35 -25.4) (size 1.7 1.7) (drill 1) (layers *.Cu *.Mask) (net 72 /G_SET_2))
  (pad 6 thru_hole circle (at 8.89 -25.4) (size 1.7 1.7) (drill 1) (layers *.Cu *.Mask) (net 74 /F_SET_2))
  (pad 5 thru_hole circle (at 11.43 -25.4) (size 1.7 1.7) (drill 1) (layers *.Cu *.Mask) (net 79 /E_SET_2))
  (pad 4 thru_hole circle (at 13.97 -25.4) (size 1.7 1.7) (drill 1) (layers *.Cu *.Mask) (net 80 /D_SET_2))
  (pad 3 thru_hole circle (at 16.51 -25.4) (size 1.7 1.7) (drill 1) (layers *.Cu *.Mask) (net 82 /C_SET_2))
  (pad 2 thru_hole circle (at 19.05 -25.4) (size 1.7 1.7) (drill 1) (layers *.Cu *.Mask) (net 83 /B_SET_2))
  (pad 1 thru_hole rect (at 21.59 -25.4) (size 1.7 1.7) (drill 1) (layers *.Cu *.Mask) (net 81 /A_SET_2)))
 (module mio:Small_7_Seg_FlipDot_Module (layer F.Cu) (at 173.2915 116.205)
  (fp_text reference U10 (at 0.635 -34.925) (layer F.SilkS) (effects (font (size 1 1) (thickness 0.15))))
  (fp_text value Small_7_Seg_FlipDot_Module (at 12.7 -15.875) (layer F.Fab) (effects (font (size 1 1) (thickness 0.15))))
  (pad 15 thru_hole circle (at 3.81 -6.35) (size 1.7 1.7) (drill 1) (layers *.Cu *.Mask) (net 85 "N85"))
  (pad 14 thru_hole circle (at 6.35 -6.35) (size 1.7 1.7) (drill 1) (layers *.Cu *.Mask) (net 65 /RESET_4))
  (pad 13 thru_hole circle (at 8.89 -6.35) (size 1.7 1.7) (drill 1) (layers *.Cu *.Mask) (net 65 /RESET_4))
  (pad 12 thru_hole circle (at 11.43 -6.35) (size 1.7 1.7) (drill 1) (layers *.Cu *.Mask) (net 65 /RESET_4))
  (pad 11 thru_hole circle (at 13.97 -6.35) (size 1.7 1.7) (drill 1) (layers *.Cu *.Mask) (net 65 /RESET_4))
  (pad 10 thru_hole circle (at 16.51 -6.35) (size 1.7 1.7) (drill 1) (layers *.Cu *.Mask) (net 65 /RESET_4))
  (pad 9 thru_hole circle (at 19.05 -6.35) (size 1.7 1.7) (drill 1) (layers *.Cu *.Mask) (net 65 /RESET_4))
  (pad 8 thru_hole rect (at 21.59 -6.35) (size 1.7 1.7) (drill 1) (layers *.Cu *.Mask) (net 65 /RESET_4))
  (pad 7 thru_hole circle (at 6.35 -25.4) (size 1.7 1.7) (drill 1) (layers *.Cu *.Mask) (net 63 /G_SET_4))
  (pad 6 thru_hole circle (at 8.89 -25.4) (size 1.7 1.7) (drill 1) (layers *.Cu *.Mask) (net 58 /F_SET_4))
  (pad 5 thru_hole circle (at 11.43 -25.4) (size 1.7 1.7) (drill 1) (layers *.Cu *.Mask) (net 64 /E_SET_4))
  (pad 4 thru_hole circle (at 13.97 -25.4) (size 1.7 1.7) (drill 1) (layers *.Cu *.Mask) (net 56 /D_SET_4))
  (pad 3 thru_hole circle (at 16.51 -25.4) (size 1.7 1.7) (drill 1) (layers *.Cu *.Mask) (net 57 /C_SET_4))
  (pad 2 thru_hole circle (at 19.05 -25.4) (size 1.7 1.7) (drill 1) (layers *.Cu *.Mask) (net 67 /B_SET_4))
  (pad 1 thru_hole rect (at 21.59 -25.4) (size 1.7 1.7) (drill 1) (layers *.Cu *.Mask) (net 66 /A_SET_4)))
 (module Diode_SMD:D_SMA (layer F.Cu) (at 96.488 105.283)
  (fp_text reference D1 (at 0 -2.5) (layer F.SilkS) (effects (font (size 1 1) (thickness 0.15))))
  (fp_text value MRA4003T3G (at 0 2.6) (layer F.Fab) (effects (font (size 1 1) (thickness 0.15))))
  (pad 1 smd rect (at -2 0) (size 2.5 1.8) (layers F.Cu F.Paste F.Mask) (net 38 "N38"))
  (pad 2 smd rect (at 2 0) (size 2.5 1.8) (layers F.Cu F.Paste F.Mask) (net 1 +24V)))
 (gr_line (start 78.486 120.904) (end 78.486 77.47) (layer Edge.Cuts) (width 0.05))
 (gr_line (start 216.916 120.904) (end 78.486 120.904) (layer Edge.Cuts) (width 0.05))
 (gr_line (start 216.916 77.47) (end 216.916 120.904) (layer Edge.Cuts) (width 0.05))
 (gr_line (start 78.486 77.47) (end 216.916 77.47) (layer Edge.Cuts) (width 0.05))
 (segment (start 95.25 90.805) (end 90.81771 95.23729) (width 0.381) (layer F.Cu) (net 42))
 (segment (start 83.831 101.357) (end 84.9415 101.357) (width 0.381) (layer F.Cu) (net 42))
 (segment (start 83.388589 100.914589) (end 83.831 101.357) (width 0.381) (layer F.Cu) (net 42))
 (segment (start 83.388589 99.300052) (end 83.388589 100.914589) (width 0.381) (layer F.Cu) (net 42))
 (segment (start 87.451351 95.23729) (end 83.388589 99.300052) (width 0.381) (layer F.Cu) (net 42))
 (segment (start 90.81771 95.23729) (end 87.451351 95.23729) (width 0.381) (layer F.Cu) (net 42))
 (segment (start 83.972799 99.542039) (end 87.693338 95.8215) (width 0.381) (layer F.Cu) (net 44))
 (segment (start 84.107838 100.707) (end 83.972799 100.571961) (width 0.381) (layer F.Cu) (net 44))
 (segment (start 83.972799 100.571961) (end 83.972799 99.542039) (width 0.381) (layer F.Cu) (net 44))
 (segment (start 84.9415 100.707) (end 84.107838 100.707) (width 0.381) (layer F.Cu) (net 44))
 (segment (start 92.7735 95.8215) (end 97.79 90.805) (width 0.381) (layer F.Cu) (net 44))
 (segment (start 87.693338 95.8215) (end 92.7735 95.8215) (width 0.381) (layer F.Cu) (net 44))
 (segment (start 83.9855 105.907) (end 84.9415 105.907) (width 0.381) (layer F.Cu) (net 35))
 (segment (start 82.220169 104.141669) (end 83.9855 105.907) (width 0.381) (layer F.Cu) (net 35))
 (segment (start 82.220169 98.754831) (end 82.220169 104.141669) (width 0.381) (layer F.Cu) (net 35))
 (segment (start 90.17 90.805) (end 82.220169 98.754831) (width 0.381) (layer F.Cu) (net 35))
 (segment (start 83.5065 106.557) (end 84.9415 106.557) (width 0.381) (layer F.Cu) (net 33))
 (segment (start 81.635959 104.686459) (end 83.5065 106.557) (width 0.381) (layer F.Cu) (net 33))
 (segment (start 81.635959 96.799041) (end 81.635959 104.686459) (width 0.381) (layer F.Cu) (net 33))
 (segment (start 87.63 90.805) (end 81.635959 96.799041) (width 0.381) (layer F.Cu) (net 33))
 (segment (start 92.71 90.805) (end 88.86192 94.65308) (width 0.381) (layer F.Cu) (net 41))
 (segment (start 83.465 102.007) (end 84.9415 102.007) (width 0.381) (layer F.Cu) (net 41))
 (segment (start 82.804379 101.346379) (end 83.465 102.007) (width 0.381) (layer F.Cu) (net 41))
 (segment (start 82.804379 99.058065) (end 82.804379 101.346379) (width 0.381) (layer F.Cu) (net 41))
 (segment (start 87.209364 94.65308) (end 82.804379 99.058065) (width 0.381) (layer F.Cu) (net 41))
 (segment (start 88.86192 94.65308) (end 87.209364 94.65308) (width 0.381) (layer F.Cu) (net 41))
 (segment (start 91.952 106.557) (end 95.25 109.855) (width 0.381) (layer F.Cu) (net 34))
 (segment (start 90.1915 106.557) (end 91.952 106.557) (width 0.381) (layer F.Cu) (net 34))
 (segment (start 95.25 109.855) (end 92.71 109.855) (width 0.381) (layer F.Cu) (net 34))
 (segment (start 92.71 109.855) (end 90.17 109.855) (width 0.381) (layer F.Cu) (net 34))
 (segment (start 90.17 109.855) (end 87.63 109.855) (width 0.381) (layer F.Cu) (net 34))
 (segment (start 95.25 109.855) (end 97.79 109.855) (width 0.381) (layer F.Cu) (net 34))
 (segment (start 97.79 109.855) (end 100.33 109.855) (width 0.381) (layer F.Cu) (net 34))
 (segment (start 100.33 109.855) (end 102.87 109.855) (width 0.381) (layer F.Cu) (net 34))
 (segment (start 91.323696 101.357) (end 93.94192 98.738777) (width 0.381) (layer F.Cu) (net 43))
 (segment (start 90.1915 101.357) (end 91.323696 101.357) (width 0.381) (layer F.Cu) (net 43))
 (segment (start 93.94192 98.738777) (end 93.94192 96.812776) (width 0.381) (layer F.Cu) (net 43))
 (segment (start 101.042089 92.632911) (end 102.87 90.805) (width 0.381) (layer F.Cu) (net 43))
 (segment (start 98.121785 92.632911) (end 101.042089 92.632911) (width 0.381) (layer F.Cu) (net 43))
 (segment (start 93.94192 96.812776) (end 98.121785 92.632911) (width 0.381) (layer F.Cu) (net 43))
 (segment (start 91.1475 100.707) (end 93.35771 98.49679) (width 0.381) (layer F.Cu) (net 45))
 (segment (start 90.1915 100.707) (end 91.1475 100.707) (width 0.381) (layer F.Cu) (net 45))
 (segment (start 99.086299 92.048701) (end 100.33 90.805) (width 0.381) (layer F.Cu) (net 45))
 (segment (start 97.879799 92.048701) (end 99.086299 92.048701) (width 0.381) (layer F.Cu) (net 45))
 (segment (start 93.35771 96.57079) (end 97.879799 92.048701) (width 0.381) (layer F.Cu) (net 45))
 (segment (start 93.35771 98.49679) (end 93.35771 96.57079) (width 0.381) (layer F.Cu) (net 45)))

